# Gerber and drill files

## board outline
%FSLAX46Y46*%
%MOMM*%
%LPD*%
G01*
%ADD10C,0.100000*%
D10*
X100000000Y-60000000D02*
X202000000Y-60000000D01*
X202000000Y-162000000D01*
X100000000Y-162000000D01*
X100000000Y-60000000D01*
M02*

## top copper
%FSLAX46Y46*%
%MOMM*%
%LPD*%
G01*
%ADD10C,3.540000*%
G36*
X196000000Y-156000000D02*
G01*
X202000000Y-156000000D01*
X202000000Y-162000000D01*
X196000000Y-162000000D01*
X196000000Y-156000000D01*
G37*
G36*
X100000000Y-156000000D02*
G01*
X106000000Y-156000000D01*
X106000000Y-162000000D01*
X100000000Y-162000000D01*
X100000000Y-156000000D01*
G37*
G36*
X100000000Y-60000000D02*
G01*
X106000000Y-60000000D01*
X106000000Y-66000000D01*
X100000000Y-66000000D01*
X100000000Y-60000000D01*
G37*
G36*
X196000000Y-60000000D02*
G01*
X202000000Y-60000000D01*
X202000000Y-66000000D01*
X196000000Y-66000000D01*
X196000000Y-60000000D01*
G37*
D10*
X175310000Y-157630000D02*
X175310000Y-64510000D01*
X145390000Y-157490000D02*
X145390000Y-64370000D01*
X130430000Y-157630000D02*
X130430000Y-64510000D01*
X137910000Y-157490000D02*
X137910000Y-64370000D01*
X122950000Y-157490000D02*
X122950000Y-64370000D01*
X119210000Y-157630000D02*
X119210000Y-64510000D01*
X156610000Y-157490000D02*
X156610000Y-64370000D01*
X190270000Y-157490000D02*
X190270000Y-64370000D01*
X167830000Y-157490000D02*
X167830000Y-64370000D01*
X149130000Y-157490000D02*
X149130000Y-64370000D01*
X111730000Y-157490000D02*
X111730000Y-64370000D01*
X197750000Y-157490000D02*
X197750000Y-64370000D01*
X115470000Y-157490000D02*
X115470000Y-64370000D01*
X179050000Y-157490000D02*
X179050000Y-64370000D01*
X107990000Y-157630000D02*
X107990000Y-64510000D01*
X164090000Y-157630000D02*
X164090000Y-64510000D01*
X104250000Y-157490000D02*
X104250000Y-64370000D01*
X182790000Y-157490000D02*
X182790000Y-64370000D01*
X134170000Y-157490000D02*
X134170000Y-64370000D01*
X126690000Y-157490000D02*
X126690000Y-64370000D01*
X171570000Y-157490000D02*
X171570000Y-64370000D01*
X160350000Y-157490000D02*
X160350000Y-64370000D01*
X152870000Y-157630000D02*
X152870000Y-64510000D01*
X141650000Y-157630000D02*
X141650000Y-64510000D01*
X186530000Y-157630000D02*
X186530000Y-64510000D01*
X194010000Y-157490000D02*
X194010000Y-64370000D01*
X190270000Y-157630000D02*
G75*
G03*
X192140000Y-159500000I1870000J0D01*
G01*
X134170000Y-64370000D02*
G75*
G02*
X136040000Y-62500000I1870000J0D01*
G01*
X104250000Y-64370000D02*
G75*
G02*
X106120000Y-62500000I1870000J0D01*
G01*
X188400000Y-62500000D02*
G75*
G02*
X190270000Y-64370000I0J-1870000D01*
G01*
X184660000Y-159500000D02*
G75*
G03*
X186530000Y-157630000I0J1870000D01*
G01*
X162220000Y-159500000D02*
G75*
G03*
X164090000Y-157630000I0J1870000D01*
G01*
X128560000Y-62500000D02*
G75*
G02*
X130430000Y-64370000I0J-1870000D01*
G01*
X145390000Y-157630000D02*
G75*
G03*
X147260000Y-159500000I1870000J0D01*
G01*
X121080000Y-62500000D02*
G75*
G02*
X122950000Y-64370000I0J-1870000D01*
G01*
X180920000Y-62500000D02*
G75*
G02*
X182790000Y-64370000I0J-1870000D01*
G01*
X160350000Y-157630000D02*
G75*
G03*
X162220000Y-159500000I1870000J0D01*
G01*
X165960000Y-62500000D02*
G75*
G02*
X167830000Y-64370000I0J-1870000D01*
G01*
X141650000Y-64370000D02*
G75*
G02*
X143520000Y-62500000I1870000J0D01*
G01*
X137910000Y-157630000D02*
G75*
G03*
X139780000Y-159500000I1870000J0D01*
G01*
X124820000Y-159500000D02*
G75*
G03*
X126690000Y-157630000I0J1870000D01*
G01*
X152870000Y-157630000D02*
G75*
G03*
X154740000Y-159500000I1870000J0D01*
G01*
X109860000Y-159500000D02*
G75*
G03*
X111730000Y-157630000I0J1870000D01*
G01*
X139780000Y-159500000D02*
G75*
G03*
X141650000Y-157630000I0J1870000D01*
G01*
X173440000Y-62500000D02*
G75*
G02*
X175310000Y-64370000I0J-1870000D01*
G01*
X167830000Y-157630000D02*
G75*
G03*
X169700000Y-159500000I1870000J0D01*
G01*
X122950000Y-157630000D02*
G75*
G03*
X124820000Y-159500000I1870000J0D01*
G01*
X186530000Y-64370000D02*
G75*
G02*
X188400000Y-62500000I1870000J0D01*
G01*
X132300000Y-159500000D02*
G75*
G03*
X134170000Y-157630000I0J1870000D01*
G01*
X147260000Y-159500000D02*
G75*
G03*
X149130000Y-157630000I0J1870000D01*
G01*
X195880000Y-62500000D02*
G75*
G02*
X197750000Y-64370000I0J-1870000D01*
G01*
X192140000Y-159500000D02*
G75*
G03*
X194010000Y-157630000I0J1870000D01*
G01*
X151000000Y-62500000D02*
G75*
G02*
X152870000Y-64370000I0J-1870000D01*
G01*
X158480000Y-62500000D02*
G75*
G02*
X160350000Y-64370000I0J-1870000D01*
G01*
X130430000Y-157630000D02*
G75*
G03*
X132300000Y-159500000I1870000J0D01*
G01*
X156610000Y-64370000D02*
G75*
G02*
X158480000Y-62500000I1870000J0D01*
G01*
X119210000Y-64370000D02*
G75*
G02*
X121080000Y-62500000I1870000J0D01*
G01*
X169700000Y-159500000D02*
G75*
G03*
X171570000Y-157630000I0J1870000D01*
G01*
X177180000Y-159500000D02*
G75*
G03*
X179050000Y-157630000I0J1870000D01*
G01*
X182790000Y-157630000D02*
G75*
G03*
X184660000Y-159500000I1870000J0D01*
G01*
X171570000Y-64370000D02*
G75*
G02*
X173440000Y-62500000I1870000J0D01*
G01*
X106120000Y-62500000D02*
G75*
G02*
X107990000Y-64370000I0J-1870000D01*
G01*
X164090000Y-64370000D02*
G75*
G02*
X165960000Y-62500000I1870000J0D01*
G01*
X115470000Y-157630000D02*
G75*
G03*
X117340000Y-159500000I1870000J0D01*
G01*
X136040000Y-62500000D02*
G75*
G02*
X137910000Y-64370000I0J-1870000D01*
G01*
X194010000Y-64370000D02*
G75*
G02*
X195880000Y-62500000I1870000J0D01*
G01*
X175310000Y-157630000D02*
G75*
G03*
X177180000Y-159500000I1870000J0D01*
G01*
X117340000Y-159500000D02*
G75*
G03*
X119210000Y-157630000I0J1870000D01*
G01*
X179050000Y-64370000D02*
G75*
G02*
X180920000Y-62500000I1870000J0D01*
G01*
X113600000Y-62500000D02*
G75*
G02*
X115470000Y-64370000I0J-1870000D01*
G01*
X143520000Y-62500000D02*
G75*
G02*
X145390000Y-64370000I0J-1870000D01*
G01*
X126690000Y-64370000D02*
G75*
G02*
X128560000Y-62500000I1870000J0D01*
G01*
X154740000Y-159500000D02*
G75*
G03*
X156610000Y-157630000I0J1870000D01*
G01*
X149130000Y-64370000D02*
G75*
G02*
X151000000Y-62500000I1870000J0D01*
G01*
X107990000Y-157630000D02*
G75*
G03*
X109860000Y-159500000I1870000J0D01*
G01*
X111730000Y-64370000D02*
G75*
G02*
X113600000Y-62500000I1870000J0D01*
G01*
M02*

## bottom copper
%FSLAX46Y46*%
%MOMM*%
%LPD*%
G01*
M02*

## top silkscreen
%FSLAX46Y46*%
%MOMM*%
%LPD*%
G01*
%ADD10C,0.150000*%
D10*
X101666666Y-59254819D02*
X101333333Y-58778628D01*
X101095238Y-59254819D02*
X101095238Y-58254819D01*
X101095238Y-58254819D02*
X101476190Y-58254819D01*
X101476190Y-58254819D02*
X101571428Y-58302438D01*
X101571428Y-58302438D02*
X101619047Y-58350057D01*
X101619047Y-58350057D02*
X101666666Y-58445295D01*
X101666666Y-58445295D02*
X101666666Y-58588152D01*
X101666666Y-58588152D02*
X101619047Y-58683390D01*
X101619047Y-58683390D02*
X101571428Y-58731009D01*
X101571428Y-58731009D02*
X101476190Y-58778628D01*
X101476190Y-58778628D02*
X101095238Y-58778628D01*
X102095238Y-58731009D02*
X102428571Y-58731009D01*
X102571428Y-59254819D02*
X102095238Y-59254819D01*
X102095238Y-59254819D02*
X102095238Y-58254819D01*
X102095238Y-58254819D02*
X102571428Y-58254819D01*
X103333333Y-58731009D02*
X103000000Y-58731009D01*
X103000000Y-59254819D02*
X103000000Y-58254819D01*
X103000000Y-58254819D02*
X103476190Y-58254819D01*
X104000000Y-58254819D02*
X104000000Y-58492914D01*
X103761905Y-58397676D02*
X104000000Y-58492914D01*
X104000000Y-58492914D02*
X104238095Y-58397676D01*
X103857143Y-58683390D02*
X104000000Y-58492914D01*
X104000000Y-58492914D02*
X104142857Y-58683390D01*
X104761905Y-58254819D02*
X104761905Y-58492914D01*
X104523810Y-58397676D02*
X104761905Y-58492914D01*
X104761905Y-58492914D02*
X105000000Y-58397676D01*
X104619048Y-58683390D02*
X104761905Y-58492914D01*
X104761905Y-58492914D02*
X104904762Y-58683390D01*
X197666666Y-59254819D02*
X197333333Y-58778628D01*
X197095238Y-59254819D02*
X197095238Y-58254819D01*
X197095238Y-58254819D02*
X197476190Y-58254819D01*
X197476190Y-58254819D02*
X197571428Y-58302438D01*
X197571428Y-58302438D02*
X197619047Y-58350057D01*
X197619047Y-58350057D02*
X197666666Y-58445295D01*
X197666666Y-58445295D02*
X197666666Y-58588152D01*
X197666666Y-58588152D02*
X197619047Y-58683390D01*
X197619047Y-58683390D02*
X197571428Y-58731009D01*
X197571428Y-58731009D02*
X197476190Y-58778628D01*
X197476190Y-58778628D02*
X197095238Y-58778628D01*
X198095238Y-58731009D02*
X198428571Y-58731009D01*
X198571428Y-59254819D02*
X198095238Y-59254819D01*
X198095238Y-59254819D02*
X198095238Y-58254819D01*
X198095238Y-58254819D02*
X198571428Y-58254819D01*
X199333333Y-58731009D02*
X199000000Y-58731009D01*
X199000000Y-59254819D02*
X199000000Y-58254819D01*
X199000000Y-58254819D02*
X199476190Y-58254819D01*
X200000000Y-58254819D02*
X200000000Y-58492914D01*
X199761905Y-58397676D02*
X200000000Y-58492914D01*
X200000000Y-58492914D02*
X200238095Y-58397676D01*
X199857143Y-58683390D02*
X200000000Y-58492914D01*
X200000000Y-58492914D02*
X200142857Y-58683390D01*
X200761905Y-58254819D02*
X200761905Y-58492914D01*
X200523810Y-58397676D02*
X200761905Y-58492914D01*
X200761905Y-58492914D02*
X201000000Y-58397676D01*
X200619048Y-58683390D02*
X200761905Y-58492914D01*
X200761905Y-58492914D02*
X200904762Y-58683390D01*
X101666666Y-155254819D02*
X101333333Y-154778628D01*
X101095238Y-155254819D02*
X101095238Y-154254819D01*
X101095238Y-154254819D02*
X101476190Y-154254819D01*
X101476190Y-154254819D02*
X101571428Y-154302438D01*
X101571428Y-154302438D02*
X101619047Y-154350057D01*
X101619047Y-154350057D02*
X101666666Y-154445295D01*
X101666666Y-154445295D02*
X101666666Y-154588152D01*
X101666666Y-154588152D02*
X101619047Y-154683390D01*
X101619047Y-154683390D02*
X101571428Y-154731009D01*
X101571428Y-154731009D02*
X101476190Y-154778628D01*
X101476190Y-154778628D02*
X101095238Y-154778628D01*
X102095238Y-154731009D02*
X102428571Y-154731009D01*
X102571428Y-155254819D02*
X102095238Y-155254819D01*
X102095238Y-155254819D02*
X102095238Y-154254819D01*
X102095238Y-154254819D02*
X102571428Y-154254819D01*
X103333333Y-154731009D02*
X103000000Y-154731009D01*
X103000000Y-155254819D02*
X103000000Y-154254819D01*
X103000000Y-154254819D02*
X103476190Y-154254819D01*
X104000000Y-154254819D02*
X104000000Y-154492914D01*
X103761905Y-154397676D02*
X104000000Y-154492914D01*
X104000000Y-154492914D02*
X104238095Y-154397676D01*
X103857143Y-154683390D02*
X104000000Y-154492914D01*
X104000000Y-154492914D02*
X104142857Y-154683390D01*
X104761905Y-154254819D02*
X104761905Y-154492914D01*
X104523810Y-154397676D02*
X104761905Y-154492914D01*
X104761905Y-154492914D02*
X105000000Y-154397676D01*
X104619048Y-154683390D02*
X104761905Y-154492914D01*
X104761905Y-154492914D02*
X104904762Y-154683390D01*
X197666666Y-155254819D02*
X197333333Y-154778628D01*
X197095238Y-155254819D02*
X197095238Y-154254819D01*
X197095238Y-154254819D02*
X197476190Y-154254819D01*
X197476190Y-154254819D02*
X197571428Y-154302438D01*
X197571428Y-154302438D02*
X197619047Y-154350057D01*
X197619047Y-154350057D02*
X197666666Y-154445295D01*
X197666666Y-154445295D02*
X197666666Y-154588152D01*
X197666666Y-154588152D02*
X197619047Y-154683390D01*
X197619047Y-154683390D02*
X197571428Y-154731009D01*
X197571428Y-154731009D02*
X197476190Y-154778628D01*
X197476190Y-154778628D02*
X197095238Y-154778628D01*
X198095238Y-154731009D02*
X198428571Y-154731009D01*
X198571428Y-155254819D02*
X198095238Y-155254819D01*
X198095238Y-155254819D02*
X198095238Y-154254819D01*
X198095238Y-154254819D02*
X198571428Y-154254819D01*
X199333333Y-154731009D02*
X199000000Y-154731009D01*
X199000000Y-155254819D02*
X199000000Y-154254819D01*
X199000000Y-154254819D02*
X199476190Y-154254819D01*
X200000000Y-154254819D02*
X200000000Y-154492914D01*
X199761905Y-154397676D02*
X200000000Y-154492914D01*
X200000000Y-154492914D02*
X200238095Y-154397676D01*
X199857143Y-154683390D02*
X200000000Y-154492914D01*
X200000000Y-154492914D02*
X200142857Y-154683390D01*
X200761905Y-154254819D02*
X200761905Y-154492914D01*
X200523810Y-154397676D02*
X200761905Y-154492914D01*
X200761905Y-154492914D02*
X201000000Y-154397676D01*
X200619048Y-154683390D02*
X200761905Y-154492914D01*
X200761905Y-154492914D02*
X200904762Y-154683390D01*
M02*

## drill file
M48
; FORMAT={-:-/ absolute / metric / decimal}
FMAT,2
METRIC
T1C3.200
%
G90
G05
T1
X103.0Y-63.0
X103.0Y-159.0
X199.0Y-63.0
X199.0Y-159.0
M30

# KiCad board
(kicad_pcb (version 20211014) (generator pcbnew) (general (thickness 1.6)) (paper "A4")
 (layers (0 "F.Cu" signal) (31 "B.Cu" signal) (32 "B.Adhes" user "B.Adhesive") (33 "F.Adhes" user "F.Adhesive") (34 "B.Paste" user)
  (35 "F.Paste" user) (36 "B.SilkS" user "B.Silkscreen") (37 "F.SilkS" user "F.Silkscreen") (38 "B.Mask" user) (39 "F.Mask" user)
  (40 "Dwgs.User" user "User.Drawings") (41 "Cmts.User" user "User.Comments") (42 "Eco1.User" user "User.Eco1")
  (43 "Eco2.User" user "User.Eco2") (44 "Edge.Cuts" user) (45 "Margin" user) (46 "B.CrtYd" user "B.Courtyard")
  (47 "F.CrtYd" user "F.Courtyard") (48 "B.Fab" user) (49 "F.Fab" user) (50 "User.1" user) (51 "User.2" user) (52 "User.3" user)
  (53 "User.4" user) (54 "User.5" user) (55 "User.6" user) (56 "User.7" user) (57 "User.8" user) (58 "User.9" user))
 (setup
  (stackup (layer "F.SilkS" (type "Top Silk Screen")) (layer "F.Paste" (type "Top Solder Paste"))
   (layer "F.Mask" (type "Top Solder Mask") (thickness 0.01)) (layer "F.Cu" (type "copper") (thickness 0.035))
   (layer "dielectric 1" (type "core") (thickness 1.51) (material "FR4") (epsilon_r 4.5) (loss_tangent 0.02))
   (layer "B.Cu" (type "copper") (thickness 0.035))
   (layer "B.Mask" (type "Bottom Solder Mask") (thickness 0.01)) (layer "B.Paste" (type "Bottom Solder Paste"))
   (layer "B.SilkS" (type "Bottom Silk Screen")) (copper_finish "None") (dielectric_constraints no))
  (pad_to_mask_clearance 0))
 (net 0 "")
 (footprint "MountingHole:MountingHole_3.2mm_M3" (layer "F.Cu") (at 103 63)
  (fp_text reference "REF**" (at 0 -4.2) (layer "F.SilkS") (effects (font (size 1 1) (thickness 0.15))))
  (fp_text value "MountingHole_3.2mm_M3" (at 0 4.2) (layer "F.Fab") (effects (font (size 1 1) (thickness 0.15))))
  (pad "" np_thru_hole circle (at 0 0) (size 3.2 3.2) (drill 3.2) (layers *.Cu *.Mask)))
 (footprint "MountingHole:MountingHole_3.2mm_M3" (layer "F.Cu") (at 199 63)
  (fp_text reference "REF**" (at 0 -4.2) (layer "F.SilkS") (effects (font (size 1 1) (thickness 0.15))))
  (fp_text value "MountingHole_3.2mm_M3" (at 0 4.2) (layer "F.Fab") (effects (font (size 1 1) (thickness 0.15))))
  (pad "" np_thru_hole circle (at 0 0) (size 3.2 3.2) (drill 3.2) (layers *.Cu *.Mask)))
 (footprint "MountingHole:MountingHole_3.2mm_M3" (layer "F.Cu") (at 103 159)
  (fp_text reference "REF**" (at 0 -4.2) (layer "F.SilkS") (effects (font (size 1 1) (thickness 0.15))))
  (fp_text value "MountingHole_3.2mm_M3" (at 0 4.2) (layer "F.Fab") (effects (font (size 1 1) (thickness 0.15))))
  (pad "" np_thru_hole circle (at 0 0) (size 3.2 3.2) (drill 3.2) (layers *.Cu *.Mask)))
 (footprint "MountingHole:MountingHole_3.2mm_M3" (layer "F.Cu") (at 199 159)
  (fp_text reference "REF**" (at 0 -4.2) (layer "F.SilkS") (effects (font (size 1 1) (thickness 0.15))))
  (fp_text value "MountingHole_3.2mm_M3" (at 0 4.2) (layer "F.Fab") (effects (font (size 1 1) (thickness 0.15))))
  (pad "" np_thru_hole circle (at 0 0) (size 3.2 3.2) (drill 3.2) (layers *.Cu *.Mask)))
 (gr_rect (start 202 162) (end 196 156) (layer "F.Cu") (width 0) (fill solid))
 (gr_rect (start 106 156) (end 100 162) (layer "F.Cu") (width 0) (fill solid))
 (gr_rect (start 106 66) (end 100 60) (layer "F.Cu") (width 0) (fill solid))
 (gr_rect (start 202 66) (end 196 60) (layer "F.Cu") (width 0) (fill solid))
 (gr_rect (start 100 60) (end 202 162) (layer "Edge.Cuts") (width 0.1) (fill none))
 (segment (start 175.31 157.63) (end 175.31 64.51) (width 3.54) (layer "F.Cu") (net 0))
 (segment (start 145.39 157.49) (end 145.39 64.37) (width 3.54) (layer "F.Cu") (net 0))
 (segment (start 130.43 157.63) (end 130.43 64.51) (width 3.54) (layer "F.Cu") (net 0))
 (segment (start 137.91 157.49) (end 137.91 64.37) (width 3.54) (layer "F.Cu") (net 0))
 (segment (start 122.95 157.49) (end 122.95 64.37) (width 3.54) (layer "F.Cu") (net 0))
 (segment (start 119.21 157.63) (end 119.21 64.51) (width 3.54) (layer "F.Cu") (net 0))
 (segment (start 156.61 157.49) (end 156.61 64.37) (width 3.54) (layer "F.Cu") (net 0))
 (segment (start 190.27 157.49) (end 190.27 64.37) (width 3.54) (layer "F.Cu") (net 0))
 (segment (start 167.83 157.49) (end 167.83 64.37) (width 3.54) (layer "F.Cu") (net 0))
 (segment (start 149.13 157.49) (end 149.13 64.37) (width 3.54) (layer "F.Cu") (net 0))
 (segment (start 111.73 157.49) (end 111.73 64.37) (width 3.54) (layer "F.Cu") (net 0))
 (segment (start 197.75 157.49) (end 197.75 64.37) (width 3.54) (layer "F.Cu") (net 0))
 (segment (start 115.47 157.49) (end 115.47 64.37) (width 3.54) (layer "F.Cu") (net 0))
 (segment (start 179.05 157.49) (end 179.05 64.37) (width 3.54) (layer "F.Cu") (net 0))
 (segment (start 107.99 157.63) (end 107.99 64.51) (width 3.54) (layer "F.Cu") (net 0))
 (segment (start 164.09 157.63) (end 164.09 64.51) (width 3.54) (layer "F.Cu") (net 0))
 (segment (start 104.25 157.49) (end 104.25 64.37) (width 3.54) (layer "F.Cu") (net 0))
 (segment (start 182.79 157.49) (end 182.79 64.37) (width 3.54) (layer "F.Cu") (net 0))
 (segment (start 134.17 157.49) (end 134.17 64.37) (width 3.54) (layer "F.Cu") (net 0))
 (segment (start 126.69 157.49) (end 126.69 64.37) (width 3.54) (layer "F.Cu") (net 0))
 (segment (start 171.57 157.49) (end 171.57 64.37) (width 3.54) (layer "F.Cu") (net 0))
 (segment (start 160.35 157.49) (end 160.35 64.37) (width 3.54) (layer "F.Cu") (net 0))
 (segment (start 152.87 157.63) (end 152.87 64.51) (width 3.54) (layer "F.Cu") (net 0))
 (segment (start 141.65 157.63) (end 141.65 64.51) (width 3.54) (layer "F.Cu") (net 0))
 (segment (start 186.53 157.63) (end 186.53 64.51) (width 3.54) (layer "F.Cu") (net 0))
 (segment (start 194.01 157.49) (end 194.01 64.37) (width 3.54) (layer "F.Cu") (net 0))
 (arc (start 190.27 157.63) (mid 190.81771 158.95229) (end 192.14 159.5) (width 3.54) (layer "F.Cu") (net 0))
 (arc (start 134.17 64.37) (mid 134.71771 63.04771) (end 136.04 62.5) (width 3.54) (layer "F.Cu") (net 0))
 (arc (start 104.25 64.37) (mid 104.79771 63.04771) (end 106.12 62.5) (width 3.54) (layer "F.Cu") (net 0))
 (arc (start 188.4 62.5) (mid 189.72229 63.04771) (end 190.27 64.37) (width 3.54) (layer "F.Cu") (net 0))
 (arc (start 184.66 159.5) (mid 185.98229 158.95229) (end 186.53 157.63) (width 3.54) (layer "F.Cu") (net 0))
 (arc (start 162.22 159.5) (mid 163.54229 158.95229) (end 164.09 157.63) (width 3.54) (layer "F.Cu") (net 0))
 (arc (start 128.56 62.5) (mid 129.88229 63.04771) (end 130.43 64.37) (width 3.54) (layer "F.Cu") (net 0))
 (arc (start 145.39 157.63) (mid 145.93771 158.95229) (end 147.26 159.5) (width 3.54) (layer "F.Cu") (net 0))
 (arc (start 121.08 62.5) (mid 122.40229 63.04771) (end 122.95 64.37) (width 3.54) (layer "F.Cu") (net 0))
 (arc (start 180.92 62.5) (mid 182.24229 63.04771) (end 182.79 64.37) (width 3.54) (layer "F.Cu") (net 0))
 (arc (start 160.35 157.63) (mid 160.89771 158.95229) (end 162.22 159.5) (width 3.54) (layer "F.Cu") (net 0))
 (arc (start 165.96 62.5) (mid 167.28229 63.04771) (end 167.83 64.37) (width 3.54) (layer "F.Cu") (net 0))
 (arc (start 141.65 64.37) (mid 142.19771 63.04771) (end 143.52 62.5) (width 3.54) (layer "F.Cu") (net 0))
 (arc (start 137.91 157.63) (mid 138.45771 158.95229) (end 139.78 159.5) (width 3.54) (layer "F.Cu") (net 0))
 (arc (start 124.82 159.5) (mid 126.14229 158.95229) (end 126.69 157.63) (width 3.54) (layer "F.Cu") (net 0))
 (arc (start 152.87 157.63) (mid 153.41771 158.95229) (end 154.74 159.5) (width 3.54) (layer "F.Cu") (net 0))
 (arc (start 109.86 159.5) (mid 111.18229 158.95229) (end 111.73 157.63) (width 3.54) (layer "F.Cu") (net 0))
 (arc (start 139.78 159.5) (mid 141.10229 158.95229) (end 141.65 157.63) (width 3.54) (layer "F.Cu") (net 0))
 (arc (start 173.44 62.5) (mid 174.76229 63.04771) (end 175.31 64.37) (width 3.54) (layer "F.Cu") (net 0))
 (arc (start 167.83 157.63) (mid 168.37771 158.95229) (end 169.7 159.5) (width 3.54) (layer "F.Cu") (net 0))
 (arc (start 122.95 157.63) (mid 123.49771 158.95229) (end 124.82 159.5) (width 3.54) (layer "F.Cu") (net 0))
 (arc (start 186.53 64.37) (mid 187.07771 63.04771) (end 188.4 62.5) (width 3.54) (layer "F.Cu") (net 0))
 (arc (start 132.3 159.5) (mid 133.62229 158.95229) (end 134.17 157.63) (width 3.54) (layer "F.Cu") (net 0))
 (arc (start 147.26 159.5) (mid 148.58229 158.95229) (end 149.13 157.63) (width 3.54) (layer "F.Cu") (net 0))
 (arc (start 195.88 62.5) (mid 197.20229 63.04771) (end 197.75 64.37) (width 3.54) (layer "F.Cu") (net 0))
 (arc (start 192.14 159.5) (mid 193.46229 158.95229) (end 194.01 157.63) (width 3.54) (layer "F.Cu") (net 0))
 (arc (start 151 62.5) (mid 152.32229 63.04771) (end 152.87 64.37) (width 3.54) (layer "F.Cu") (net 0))
 (arc (start 158.48 62.5) (mid 159.80229 63.04771) (end 160.35 64.37) (width 3.54) (layer "F.Cu") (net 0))
 (arc (start 130.43 157.63) (mid 130.97771 158.95229) (end 132.3 159.5) (width 3.54) (layer "F.Cu") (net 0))
 (arc (start 156.61 64.37) (mid 157.15771 63.04771) (end 158.48 62.5) (width 3.54) (layer "F.Cu") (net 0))
 (arc (start 119.21 64.37) (mid 119.75771 63.04771) (end 121.08 62.5) (width 3.54) (layer "F.Cu") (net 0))
 (arc (start 169.7 159.5) (mid 171.02229 158.95229) (end 171.57 157.63) (width 3.54) (layer "F.Cu") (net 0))
 (arc (start 177.18 159.5) (mid 178.50229 158.95229) (end 179.05 157.63) (width 3.54) (layer "F.Cu") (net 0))
 (arc (start 182.79 157.63) (mid 183.33771 158.95229) (end 184.66 159.5) (width 3.54) (layer "F.Cu") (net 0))
 (arc (start 171.57 64.37) (mid 172.11771 63.04771) (end 173.44 62.5) (width 3.54) (layer "F.Cu") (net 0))
 (arc (start 106.12 62.5) (mid 107.44229 63.04771) (end 107.99 64.37) (width 3.54) (layer "F.Cu") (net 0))
 (arc (start 164.09 64.37) (mid 164.63771 63.04771) (end 165.96 62.5) (width 3.54) (layer "F.Cu") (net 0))
 (arc (start 115.47 157.63) (mid 116.01771 158.95229) (end 117.34 159.5) (width 3.54) (layer "F.Cu") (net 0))
 (arc (start 136.04 62.5) (mid 137.36229 63.04771) (end 137.91 64.37) (width 3.54) (layer "F.Cu") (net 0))
 (arc (start 194.01 64.37) (mid 194.55771 63.04771) (end 195.88 62.5) (width 3.54) (layer "F.Cu") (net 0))
 (arc (start 175.31 157.63) (mid 175.85771 158.95229) (end 177.18 159.5) (width 3.54) (layer "F.Cu") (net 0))
 (arc (start 117.34 159.5) (mid 118.66229 158.95229) (end 119.21 157.63) (width 3.54) (layer "F.Cu") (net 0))
 (arc (start 179.05 64.37) (mid 179.59771 63.04771) (end 180.92 62.5) (width 3.54) (layer "F.Cu") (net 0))
 (arc (start 113.6 62.5) (mid 114.92229 63.04771) (end 115.47 64.37) (width 3.54) (layer "F.Cu") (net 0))
 (arc (start 143.52 62.5) (mid 144.84229 63.04771) (end 145.39 64.37) (width 3.54) (layer "F.Cu") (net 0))
 (arc (start 126.69 64.37) (mid 127.23771 63.04771) (end 128.56 62.5) (width 3.54) (layer "F.Cu") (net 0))
 (arc (start 154.74 159.5) (mid 156.06229 158.95229) (end 156.61 157.63) (width 3.54) (layer "F.Cu") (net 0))
 (arc (start 149.13 64.37) (mid 149.67771 63.04771) (end 151 62.5) (width 3.54) (layer "F.Cu") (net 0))
 (arc (start 107.99 157.63) (mid 108.53771 158.95229) (end 109.86 159.5) (width 3.54) (layer "F.Cu") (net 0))
 (arc (start 111.73 64.37) (mid 112.27771 63.04771) (end 113.6 62.5) (width 3.54) (layer "F.Cu") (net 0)))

